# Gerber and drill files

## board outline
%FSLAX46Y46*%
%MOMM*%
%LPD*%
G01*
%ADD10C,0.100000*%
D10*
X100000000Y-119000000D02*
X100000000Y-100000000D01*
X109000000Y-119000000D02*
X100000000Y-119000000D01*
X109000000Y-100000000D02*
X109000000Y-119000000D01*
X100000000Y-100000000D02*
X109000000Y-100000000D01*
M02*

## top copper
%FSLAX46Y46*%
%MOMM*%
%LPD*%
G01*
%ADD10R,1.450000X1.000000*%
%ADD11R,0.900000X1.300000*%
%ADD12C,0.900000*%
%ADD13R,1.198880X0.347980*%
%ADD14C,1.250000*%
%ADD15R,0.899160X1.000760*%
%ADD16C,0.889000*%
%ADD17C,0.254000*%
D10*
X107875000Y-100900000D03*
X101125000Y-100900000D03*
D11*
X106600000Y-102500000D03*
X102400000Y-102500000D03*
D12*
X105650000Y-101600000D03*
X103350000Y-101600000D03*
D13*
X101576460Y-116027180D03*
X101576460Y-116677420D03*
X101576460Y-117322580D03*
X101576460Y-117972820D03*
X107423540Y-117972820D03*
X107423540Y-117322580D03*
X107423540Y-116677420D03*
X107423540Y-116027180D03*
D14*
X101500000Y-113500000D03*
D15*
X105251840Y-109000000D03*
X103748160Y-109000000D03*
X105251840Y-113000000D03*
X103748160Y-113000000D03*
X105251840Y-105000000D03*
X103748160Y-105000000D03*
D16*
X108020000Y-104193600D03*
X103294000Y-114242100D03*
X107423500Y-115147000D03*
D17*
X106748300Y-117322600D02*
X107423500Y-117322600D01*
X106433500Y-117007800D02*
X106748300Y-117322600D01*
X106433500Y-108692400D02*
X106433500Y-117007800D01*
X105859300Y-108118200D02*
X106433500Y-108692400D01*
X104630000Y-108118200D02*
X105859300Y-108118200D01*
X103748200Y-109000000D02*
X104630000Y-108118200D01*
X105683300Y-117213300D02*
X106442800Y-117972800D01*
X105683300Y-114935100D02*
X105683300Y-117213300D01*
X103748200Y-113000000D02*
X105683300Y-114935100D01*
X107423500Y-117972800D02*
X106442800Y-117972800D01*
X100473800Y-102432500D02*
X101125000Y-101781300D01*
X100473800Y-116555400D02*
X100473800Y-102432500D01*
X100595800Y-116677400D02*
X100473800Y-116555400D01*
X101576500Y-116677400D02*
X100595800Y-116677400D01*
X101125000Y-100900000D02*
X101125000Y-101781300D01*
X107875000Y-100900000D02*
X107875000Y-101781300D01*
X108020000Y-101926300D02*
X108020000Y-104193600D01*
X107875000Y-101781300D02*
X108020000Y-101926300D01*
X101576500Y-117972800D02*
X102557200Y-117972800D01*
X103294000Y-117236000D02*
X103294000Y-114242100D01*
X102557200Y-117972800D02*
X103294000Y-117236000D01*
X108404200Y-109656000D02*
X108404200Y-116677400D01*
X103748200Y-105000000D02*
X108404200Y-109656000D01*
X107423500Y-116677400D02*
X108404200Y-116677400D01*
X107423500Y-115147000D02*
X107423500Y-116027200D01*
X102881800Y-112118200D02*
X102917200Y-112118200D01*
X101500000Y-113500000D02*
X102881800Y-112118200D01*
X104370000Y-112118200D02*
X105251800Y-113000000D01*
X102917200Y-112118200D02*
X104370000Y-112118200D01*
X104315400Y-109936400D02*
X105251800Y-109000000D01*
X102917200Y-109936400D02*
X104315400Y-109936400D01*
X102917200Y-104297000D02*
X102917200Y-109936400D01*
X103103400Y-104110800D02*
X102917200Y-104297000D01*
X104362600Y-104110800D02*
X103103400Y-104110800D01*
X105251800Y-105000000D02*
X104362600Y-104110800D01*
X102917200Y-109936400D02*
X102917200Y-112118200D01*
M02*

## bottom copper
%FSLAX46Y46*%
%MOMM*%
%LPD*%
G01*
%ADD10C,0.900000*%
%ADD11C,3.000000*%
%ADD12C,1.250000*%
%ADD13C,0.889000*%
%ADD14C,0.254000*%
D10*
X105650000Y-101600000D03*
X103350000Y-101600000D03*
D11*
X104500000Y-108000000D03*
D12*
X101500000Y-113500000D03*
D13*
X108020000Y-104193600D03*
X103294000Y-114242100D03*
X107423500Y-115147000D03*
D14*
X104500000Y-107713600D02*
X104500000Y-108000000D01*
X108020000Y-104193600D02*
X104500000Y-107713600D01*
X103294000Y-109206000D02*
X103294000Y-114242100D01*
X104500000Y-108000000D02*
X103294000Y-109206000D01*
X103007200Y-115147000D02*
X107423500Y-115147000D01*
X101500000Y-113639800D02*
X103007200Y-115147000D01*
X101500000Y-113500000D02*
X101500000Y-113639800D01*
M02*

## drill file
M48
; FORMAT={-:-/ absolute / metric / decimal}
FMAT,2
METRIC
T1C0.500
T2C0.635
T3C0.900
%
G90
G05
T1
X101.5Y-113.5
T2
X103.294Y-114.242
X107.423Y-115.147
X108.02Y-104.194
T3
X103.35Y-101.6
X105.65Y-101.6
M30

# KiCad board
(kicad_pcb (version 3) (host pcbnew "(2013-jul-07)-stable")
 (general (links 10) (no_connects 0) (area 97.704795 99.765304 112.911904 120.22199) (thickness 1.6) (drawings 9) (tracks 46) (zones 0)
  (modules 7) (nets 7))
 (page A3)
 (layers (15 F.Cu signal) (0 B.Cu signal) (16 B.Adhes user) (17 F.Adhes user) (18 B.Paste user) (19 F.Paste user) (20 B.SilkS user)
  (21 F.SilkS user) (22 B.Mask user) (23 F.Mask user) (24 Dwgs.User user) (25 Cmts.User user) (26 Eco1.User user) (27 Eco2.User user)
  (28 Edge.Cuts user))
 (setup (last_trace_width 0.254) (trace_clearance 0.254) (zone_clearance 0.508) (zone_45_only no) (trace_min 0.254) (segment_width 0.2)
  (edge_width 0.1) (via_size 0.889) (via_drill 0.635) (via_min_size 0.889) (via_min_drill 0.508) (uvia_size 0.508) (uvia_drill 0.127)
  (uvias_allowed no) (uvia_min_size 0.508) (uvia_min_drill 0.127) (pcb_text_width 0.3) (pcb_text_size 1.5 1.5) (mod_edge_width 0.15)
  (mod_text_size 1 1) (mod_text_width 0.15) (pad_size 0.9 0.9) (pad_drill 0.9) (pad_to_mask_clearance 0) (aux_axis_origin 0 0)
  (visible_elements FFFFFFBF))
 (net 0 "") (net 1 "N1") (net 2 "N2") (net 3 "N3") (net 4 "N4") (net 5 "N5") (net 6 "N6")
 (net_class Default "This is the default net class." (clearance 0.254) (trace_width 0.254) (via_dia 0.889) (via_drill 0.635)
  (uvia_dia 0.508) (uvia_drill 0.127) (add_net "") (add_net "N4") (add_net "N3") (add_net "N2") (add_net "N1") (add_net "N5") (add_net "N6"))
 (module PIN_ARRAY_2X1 (layer F.Cu) (at 104.5 101.6 180)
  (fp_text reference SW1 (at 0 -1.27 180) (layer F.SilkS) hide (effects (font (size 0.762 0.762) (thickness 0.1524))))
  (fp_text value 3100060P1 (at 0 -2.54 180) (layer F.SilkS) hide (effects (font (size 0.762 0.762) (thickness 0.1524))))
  (pad 1 smd rect (at -3.375 0.7 180) (size 1.45 1) (layers F.Cu F.Paste F.Mask) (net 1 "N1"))
  (pad 2 smd rect (at 3.375 0.7 180) (size 1.45 1) (layers F.Cu F.Paste F.Mask) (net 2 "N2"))
  (pad 3 smd rect (at -2.1 -0.9 180) (size 0.9 1.3) (layers F.Cu F.Paste F.Mask))
  (pad 4 smd rect (at 2.1 -0.9 180) (size 0.9 1.3) (layers F.Cu F.Paste F.Mask))
  (pad "" thru_hole circle (at -1.15 0 180) (size 0.9 0.9) (drill 0.9) (layers *.Cu *.Mask F.SilkS))
  (pad "" thru_hole circle (at 1.15 0 180) (size 0.9 0.9) (drill 0.9) (layers *.Cu *.Mask F.SilkS)))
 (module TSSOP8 (layer F.Cu) (at 104.5 117)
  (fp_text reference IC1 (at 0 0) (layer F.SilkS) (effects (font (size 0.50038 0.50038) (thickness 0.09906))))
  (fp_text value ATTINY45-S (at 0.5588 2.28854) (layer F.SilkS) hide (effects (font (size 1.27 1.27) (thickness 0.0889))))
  (pad 1 smd rect (at -2.92354 -0.97282) (size 1.19888 0.34798) (layers F.Cu F.Paste F.Mask))
  (pad 2 smd rect (at -2.92354 -0.32258) (size 1.19888 0.34798) (layers F.Cu F.Paste F.Mask) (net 2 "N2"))
  (pad 3 smd rect (at -2.92354 0.32258) (size 1.19888 0.34798) (layers F.Cu F.Paste F.Mask))
  (pad 4 smd rect (at -2.92354 0.97282) (size 1.19888 0.34798) (layers F.Cu F.Paste F.Mask) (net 1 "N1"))
  (pad 5 smd rect (at 2.92354 0.97282) (size 1.19888 0.34798) (layers F.Cu F.Paste F.Mask) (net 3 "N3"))
  (pad 6 smd rect (at 2.92354 0.32258) (size 1.19888 0.34798) (layers F.Cu F.Paste F.Mask) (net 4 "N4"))
  (pad 7 smd rect (at 2.92354 -0.32258) (size 1.19888 0.34798) (layers F.Cu F.Paste F.Mask) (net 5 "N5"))
  (pad 8 smd rect (at 2.92354 -0.97282) (size 1.19888 0.34798) (layers F.Cu F.Paste F.Mask) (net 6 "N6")))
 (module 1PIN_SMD (layer B.Cu) (at 104.5 108)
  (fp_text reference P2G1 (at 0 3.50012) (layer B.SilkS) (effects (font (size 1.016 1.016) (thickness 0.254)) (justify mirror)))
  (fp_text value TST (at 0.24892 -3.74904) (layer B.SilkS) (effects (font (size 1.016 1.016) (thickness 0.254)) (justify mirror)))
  (pad 1 smd circle (at 0 0) (size 3 3) (layers B.Cu B.Paste B.SilkS B.Mask) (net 1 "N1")))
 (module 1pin (layer F.Cu) (at 101.5 113.5)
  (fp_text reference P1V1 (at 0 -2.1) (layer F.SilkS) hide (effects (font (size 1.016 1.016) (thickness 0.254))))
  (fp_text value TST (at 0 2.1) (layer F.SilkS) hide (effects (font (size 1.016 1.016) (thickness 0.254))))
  (pad 1 thru_hole circle (at 0 0) (size 1.25 1.25) (drill 0.5) (layers *.Cu *.Mask F.SilkS) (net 6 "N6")))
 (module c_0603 (layer F.Cu) (at 104.5 109)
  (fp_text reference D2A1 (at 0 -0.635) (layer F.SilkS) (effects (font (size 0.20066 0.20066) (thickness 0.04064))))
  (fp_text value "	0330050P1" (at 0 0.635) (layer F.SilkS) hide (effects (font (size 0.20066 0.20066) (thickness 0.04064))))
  (pad 1 smd rect (at 0.75184 0) (size 0.89916 1.00076) (layers F.Cu F.Paste F.Mask) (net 6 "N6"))
  (pad 2 smd rect (at -0.75184 0) (size 0.89916 1.00076) (layers F.Cu F.Paste F.Mask) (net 4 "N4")))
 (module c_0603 (layer F.Cu) (at 104.5 113)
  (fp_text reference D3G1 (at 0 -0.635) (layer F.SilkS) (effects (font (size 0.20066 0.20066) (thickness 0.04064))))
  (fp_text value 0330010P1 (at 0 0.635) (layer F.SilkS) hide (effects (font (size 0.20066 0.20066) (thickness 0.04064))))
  (pad 1 smd rect (at 0.75184 0) (size 0.89916 1.00076) (layers F.Cu F.Paste F.Mask) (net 6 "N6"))
  (pad 2 smd rect (at -0.75184 0) (size 0.89916 1.00076) (layers F.Cu F.Paste F.Mask) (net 3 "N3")))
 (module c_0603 (layer F.Cu) (at 104.5 105)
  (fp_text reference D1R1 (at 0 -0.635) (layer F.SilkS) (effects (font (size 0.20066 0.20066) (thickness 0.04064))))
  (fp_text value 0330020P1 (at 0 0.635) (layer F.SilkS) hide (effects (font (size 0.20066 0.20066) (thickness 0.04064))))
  (pad 1 smd rect (at 0.75184 0) (size 0.89916 1.00076) (layers F.Cu F.Paste F.Mask) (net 6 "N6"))
  (pad 2 smd rect (at -0.75184 0) (size 0.89916 1.00076) (layers F.Cu F.Paste F.Mask) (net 5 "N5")))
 (gr_line (start 100 119) (end 100 100) (angle 90) (layer Edge.Cuts) (width 0.1))
 (gr_line (start 109 119) (end 100 119) (angle 90) (layer Edge.Cuts) (width 0.1))
 (gr_line (start 109 100) (end 109 119) (angle 90) (layer Edge.Cuts) (width 0.1))
 (gr_line (start 100 100) (end 109 100) (angle 90) (layer Edge.Cuts) (width 0.1))
 (segment (start 106.7483 117.3226) (end 107.4235 117.3226) (width 0.254) (layer F.Cu) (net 4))
 (segment (start 106.4335 117.0078) (end 106.7483 117.3226) (width 0.254) (layer F.Cu) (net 4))
 (segment (start 106.4335 108.6924) (end 106.4335 117.0078) (width 0.254) (layer F.Cu) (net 4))
 (segment (start 105.8593 108.1182) (end 106.4335 108.6924) (width 0.254) (layer F.Cu) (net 4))
 (segment (start 104.63 108.1182) (end 105.8593 108.1182) (width 0.254) (layer F.Cu) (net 4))
 (segment (start 103.7482 109) (end 104.63 108.1182) (width 0.254) (layer F.Cu) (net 4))
 (segment (start 105.6833 117.2133) (end 106.4428 117.9728) (width 0.254) (layer F.Cu) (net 3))
 (segment (start 105.6833 114.9351) (end 105.6833 117.2133) (width 0.254) (layer F.Cu) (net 3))
 (segment (start 103.7482 113) (end 105.6833 114.9351) (width 0.254) (layer F.Cu) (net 3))
 (segment (start 107.4235 117.9728) (end 106.4428 117.9728) (width 0.254) (layer F.Cu) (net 3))
 (segment (start 100.4738 102.4325) (end 101.125 101.7813) (width 0.254) (layer F.Cu) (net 2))
 (segment (start 100.4738 116.5554) (end 100.4738 102.4325) (width 0.254) (layer F.Cu) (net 2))
 (segment (start 100.5958 116.6774) (end 100.4738 116.5554) (width 0.254) (layer F.Cu) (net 2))
 (segment (start 101.5765 116.6774) (end 100.5958 116.6774) (width 0.254) (layer F.Cu) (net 2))
 (segment (start 101.125 100.9) (end 101.125 101.7813) (width 0.254) (layer F.Cu) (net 2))
 (via (at 108.02 104.1936) (size 0.889) (layers F.Cu B.Cu) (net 1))
 (via (at 103.294 114.2421) (size 0.889) (layers F.Cu B.Cu) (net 1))
 (segment (start 107.875 100.9) (end 107.875 101.7813) (width 0.254) (layer F.Cu) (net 1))
 (segment (start 108.02 101.9263) (end 108.02 104.1936) (width 0.254) (layer F.Cu) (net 1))
 (segment (start 107.875 101.7813) (end 108.02 101.9263) (width 0.254) (layer F.Cu) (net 1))
 (segment (start 101.5765 117.9728) (end 102.5572 117.9728) (width 0.254) (layer F.Cu) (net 1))
 (segment (start 104.5 107.7136) (end 104.5 108) (width 0.254) (layer B.Cu) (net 1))
 (segment (start 108.02 104.1936) (end 104.5 107.7136) (width 0.254) (layer B.Cu) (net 1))
 (segment (start 103.294 109.206) (end 103.294 114.2421) (width 0.254) (layer B.Cu) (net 1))
 (segment (start 104.5 108) (end 103.294 109.206) (width 0.254) (layer B.Cu) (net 1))
 (segment (start 103.294 117.236) (end 103.294 114.2421) (width 0.254) (layer F.Cu) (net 1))
 (segment (start 102.5572 117.9728) (end 103.294 117.236) (width 0.254) (layer F.Cu) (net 1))
 (segment (start 108.4042 109.656) (end 108.4042 116.6774) (width 0.254) (layer F.Cu) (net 5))
 (segment (start 103.7482 105) (end 108.4042 109.656) (width 0.254) (layer F.Cu) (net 5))
 (segment (start 107.4235 116.6774) (end 108.4042 116.6774) (width 0.254) (layer F.Cu) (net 5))
 (via (at 107.4235 115.147) (size 0.889) (layers F.Cu B.Cu) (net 6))
 (segment (start 103.0072 115.147) (end 107.4235 115.147) (width 0.254) (layer B.Cu) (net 6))
 (segment (start 101.5 113.6398) (end 103.0072 115.147) (width 0.254) (layer B.Cu) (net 6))
 (segment (start 101.5 113.5) (end 101.5 113.6398) (width 0.254) (layer B.Cu) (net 6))
 (segment (start 107.4235 115.147) (end 107.4235 116.0272) (width 0.254) (layer F.Cu) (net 6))
 (segment (start 102.8818 112.1182) (end 102.9172 112.1182) (width 0.254) (layer F.Cu) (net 6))
 (segment (start 101.5 113.5) (end 102.8818 112.1182) (width 0.254) (layer F.Cu) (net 6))
 (segment (start 104.37 112.1182) (end 105.2518 113) (width 0.254) (layer F.Cu) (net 6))
 (segment (start 102.9172 112.1182) (end 104.37 112.1182) (width 0.254) (layer F.Cu) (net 6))
 (segment (start 104.3154 109.9364) (end 105.2518 109) (width 0.254) (layer F.Cu) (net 6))
 (segment (start 102.9172 109.9364) (end 104.3154 109.9364) (width 0.254) (layer F.Cu) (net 6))
 (segment (start 102.9172 104.297) (end 102.9172 109.9364) (width 0.254) (layer F.Cu) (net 6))
 (segment (start 103.1034 104.1108) (end 102.9172 104.297) (width 0.254) (layer F.Cu) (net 6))
 (segment (start 104.3626 104.1108) (end 103.1034 104.1108) (width 0.254) (layer F.Cu) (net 6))
 (segment (start 105.2518 105) (end 104.3626 104.1108) (width 0.254) (layer F.Cu) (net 6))
 (segment (start 102.9172 109.9364) (end 102.9172 112.1182) (width 0.254) (layer F.Cu) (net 6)))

